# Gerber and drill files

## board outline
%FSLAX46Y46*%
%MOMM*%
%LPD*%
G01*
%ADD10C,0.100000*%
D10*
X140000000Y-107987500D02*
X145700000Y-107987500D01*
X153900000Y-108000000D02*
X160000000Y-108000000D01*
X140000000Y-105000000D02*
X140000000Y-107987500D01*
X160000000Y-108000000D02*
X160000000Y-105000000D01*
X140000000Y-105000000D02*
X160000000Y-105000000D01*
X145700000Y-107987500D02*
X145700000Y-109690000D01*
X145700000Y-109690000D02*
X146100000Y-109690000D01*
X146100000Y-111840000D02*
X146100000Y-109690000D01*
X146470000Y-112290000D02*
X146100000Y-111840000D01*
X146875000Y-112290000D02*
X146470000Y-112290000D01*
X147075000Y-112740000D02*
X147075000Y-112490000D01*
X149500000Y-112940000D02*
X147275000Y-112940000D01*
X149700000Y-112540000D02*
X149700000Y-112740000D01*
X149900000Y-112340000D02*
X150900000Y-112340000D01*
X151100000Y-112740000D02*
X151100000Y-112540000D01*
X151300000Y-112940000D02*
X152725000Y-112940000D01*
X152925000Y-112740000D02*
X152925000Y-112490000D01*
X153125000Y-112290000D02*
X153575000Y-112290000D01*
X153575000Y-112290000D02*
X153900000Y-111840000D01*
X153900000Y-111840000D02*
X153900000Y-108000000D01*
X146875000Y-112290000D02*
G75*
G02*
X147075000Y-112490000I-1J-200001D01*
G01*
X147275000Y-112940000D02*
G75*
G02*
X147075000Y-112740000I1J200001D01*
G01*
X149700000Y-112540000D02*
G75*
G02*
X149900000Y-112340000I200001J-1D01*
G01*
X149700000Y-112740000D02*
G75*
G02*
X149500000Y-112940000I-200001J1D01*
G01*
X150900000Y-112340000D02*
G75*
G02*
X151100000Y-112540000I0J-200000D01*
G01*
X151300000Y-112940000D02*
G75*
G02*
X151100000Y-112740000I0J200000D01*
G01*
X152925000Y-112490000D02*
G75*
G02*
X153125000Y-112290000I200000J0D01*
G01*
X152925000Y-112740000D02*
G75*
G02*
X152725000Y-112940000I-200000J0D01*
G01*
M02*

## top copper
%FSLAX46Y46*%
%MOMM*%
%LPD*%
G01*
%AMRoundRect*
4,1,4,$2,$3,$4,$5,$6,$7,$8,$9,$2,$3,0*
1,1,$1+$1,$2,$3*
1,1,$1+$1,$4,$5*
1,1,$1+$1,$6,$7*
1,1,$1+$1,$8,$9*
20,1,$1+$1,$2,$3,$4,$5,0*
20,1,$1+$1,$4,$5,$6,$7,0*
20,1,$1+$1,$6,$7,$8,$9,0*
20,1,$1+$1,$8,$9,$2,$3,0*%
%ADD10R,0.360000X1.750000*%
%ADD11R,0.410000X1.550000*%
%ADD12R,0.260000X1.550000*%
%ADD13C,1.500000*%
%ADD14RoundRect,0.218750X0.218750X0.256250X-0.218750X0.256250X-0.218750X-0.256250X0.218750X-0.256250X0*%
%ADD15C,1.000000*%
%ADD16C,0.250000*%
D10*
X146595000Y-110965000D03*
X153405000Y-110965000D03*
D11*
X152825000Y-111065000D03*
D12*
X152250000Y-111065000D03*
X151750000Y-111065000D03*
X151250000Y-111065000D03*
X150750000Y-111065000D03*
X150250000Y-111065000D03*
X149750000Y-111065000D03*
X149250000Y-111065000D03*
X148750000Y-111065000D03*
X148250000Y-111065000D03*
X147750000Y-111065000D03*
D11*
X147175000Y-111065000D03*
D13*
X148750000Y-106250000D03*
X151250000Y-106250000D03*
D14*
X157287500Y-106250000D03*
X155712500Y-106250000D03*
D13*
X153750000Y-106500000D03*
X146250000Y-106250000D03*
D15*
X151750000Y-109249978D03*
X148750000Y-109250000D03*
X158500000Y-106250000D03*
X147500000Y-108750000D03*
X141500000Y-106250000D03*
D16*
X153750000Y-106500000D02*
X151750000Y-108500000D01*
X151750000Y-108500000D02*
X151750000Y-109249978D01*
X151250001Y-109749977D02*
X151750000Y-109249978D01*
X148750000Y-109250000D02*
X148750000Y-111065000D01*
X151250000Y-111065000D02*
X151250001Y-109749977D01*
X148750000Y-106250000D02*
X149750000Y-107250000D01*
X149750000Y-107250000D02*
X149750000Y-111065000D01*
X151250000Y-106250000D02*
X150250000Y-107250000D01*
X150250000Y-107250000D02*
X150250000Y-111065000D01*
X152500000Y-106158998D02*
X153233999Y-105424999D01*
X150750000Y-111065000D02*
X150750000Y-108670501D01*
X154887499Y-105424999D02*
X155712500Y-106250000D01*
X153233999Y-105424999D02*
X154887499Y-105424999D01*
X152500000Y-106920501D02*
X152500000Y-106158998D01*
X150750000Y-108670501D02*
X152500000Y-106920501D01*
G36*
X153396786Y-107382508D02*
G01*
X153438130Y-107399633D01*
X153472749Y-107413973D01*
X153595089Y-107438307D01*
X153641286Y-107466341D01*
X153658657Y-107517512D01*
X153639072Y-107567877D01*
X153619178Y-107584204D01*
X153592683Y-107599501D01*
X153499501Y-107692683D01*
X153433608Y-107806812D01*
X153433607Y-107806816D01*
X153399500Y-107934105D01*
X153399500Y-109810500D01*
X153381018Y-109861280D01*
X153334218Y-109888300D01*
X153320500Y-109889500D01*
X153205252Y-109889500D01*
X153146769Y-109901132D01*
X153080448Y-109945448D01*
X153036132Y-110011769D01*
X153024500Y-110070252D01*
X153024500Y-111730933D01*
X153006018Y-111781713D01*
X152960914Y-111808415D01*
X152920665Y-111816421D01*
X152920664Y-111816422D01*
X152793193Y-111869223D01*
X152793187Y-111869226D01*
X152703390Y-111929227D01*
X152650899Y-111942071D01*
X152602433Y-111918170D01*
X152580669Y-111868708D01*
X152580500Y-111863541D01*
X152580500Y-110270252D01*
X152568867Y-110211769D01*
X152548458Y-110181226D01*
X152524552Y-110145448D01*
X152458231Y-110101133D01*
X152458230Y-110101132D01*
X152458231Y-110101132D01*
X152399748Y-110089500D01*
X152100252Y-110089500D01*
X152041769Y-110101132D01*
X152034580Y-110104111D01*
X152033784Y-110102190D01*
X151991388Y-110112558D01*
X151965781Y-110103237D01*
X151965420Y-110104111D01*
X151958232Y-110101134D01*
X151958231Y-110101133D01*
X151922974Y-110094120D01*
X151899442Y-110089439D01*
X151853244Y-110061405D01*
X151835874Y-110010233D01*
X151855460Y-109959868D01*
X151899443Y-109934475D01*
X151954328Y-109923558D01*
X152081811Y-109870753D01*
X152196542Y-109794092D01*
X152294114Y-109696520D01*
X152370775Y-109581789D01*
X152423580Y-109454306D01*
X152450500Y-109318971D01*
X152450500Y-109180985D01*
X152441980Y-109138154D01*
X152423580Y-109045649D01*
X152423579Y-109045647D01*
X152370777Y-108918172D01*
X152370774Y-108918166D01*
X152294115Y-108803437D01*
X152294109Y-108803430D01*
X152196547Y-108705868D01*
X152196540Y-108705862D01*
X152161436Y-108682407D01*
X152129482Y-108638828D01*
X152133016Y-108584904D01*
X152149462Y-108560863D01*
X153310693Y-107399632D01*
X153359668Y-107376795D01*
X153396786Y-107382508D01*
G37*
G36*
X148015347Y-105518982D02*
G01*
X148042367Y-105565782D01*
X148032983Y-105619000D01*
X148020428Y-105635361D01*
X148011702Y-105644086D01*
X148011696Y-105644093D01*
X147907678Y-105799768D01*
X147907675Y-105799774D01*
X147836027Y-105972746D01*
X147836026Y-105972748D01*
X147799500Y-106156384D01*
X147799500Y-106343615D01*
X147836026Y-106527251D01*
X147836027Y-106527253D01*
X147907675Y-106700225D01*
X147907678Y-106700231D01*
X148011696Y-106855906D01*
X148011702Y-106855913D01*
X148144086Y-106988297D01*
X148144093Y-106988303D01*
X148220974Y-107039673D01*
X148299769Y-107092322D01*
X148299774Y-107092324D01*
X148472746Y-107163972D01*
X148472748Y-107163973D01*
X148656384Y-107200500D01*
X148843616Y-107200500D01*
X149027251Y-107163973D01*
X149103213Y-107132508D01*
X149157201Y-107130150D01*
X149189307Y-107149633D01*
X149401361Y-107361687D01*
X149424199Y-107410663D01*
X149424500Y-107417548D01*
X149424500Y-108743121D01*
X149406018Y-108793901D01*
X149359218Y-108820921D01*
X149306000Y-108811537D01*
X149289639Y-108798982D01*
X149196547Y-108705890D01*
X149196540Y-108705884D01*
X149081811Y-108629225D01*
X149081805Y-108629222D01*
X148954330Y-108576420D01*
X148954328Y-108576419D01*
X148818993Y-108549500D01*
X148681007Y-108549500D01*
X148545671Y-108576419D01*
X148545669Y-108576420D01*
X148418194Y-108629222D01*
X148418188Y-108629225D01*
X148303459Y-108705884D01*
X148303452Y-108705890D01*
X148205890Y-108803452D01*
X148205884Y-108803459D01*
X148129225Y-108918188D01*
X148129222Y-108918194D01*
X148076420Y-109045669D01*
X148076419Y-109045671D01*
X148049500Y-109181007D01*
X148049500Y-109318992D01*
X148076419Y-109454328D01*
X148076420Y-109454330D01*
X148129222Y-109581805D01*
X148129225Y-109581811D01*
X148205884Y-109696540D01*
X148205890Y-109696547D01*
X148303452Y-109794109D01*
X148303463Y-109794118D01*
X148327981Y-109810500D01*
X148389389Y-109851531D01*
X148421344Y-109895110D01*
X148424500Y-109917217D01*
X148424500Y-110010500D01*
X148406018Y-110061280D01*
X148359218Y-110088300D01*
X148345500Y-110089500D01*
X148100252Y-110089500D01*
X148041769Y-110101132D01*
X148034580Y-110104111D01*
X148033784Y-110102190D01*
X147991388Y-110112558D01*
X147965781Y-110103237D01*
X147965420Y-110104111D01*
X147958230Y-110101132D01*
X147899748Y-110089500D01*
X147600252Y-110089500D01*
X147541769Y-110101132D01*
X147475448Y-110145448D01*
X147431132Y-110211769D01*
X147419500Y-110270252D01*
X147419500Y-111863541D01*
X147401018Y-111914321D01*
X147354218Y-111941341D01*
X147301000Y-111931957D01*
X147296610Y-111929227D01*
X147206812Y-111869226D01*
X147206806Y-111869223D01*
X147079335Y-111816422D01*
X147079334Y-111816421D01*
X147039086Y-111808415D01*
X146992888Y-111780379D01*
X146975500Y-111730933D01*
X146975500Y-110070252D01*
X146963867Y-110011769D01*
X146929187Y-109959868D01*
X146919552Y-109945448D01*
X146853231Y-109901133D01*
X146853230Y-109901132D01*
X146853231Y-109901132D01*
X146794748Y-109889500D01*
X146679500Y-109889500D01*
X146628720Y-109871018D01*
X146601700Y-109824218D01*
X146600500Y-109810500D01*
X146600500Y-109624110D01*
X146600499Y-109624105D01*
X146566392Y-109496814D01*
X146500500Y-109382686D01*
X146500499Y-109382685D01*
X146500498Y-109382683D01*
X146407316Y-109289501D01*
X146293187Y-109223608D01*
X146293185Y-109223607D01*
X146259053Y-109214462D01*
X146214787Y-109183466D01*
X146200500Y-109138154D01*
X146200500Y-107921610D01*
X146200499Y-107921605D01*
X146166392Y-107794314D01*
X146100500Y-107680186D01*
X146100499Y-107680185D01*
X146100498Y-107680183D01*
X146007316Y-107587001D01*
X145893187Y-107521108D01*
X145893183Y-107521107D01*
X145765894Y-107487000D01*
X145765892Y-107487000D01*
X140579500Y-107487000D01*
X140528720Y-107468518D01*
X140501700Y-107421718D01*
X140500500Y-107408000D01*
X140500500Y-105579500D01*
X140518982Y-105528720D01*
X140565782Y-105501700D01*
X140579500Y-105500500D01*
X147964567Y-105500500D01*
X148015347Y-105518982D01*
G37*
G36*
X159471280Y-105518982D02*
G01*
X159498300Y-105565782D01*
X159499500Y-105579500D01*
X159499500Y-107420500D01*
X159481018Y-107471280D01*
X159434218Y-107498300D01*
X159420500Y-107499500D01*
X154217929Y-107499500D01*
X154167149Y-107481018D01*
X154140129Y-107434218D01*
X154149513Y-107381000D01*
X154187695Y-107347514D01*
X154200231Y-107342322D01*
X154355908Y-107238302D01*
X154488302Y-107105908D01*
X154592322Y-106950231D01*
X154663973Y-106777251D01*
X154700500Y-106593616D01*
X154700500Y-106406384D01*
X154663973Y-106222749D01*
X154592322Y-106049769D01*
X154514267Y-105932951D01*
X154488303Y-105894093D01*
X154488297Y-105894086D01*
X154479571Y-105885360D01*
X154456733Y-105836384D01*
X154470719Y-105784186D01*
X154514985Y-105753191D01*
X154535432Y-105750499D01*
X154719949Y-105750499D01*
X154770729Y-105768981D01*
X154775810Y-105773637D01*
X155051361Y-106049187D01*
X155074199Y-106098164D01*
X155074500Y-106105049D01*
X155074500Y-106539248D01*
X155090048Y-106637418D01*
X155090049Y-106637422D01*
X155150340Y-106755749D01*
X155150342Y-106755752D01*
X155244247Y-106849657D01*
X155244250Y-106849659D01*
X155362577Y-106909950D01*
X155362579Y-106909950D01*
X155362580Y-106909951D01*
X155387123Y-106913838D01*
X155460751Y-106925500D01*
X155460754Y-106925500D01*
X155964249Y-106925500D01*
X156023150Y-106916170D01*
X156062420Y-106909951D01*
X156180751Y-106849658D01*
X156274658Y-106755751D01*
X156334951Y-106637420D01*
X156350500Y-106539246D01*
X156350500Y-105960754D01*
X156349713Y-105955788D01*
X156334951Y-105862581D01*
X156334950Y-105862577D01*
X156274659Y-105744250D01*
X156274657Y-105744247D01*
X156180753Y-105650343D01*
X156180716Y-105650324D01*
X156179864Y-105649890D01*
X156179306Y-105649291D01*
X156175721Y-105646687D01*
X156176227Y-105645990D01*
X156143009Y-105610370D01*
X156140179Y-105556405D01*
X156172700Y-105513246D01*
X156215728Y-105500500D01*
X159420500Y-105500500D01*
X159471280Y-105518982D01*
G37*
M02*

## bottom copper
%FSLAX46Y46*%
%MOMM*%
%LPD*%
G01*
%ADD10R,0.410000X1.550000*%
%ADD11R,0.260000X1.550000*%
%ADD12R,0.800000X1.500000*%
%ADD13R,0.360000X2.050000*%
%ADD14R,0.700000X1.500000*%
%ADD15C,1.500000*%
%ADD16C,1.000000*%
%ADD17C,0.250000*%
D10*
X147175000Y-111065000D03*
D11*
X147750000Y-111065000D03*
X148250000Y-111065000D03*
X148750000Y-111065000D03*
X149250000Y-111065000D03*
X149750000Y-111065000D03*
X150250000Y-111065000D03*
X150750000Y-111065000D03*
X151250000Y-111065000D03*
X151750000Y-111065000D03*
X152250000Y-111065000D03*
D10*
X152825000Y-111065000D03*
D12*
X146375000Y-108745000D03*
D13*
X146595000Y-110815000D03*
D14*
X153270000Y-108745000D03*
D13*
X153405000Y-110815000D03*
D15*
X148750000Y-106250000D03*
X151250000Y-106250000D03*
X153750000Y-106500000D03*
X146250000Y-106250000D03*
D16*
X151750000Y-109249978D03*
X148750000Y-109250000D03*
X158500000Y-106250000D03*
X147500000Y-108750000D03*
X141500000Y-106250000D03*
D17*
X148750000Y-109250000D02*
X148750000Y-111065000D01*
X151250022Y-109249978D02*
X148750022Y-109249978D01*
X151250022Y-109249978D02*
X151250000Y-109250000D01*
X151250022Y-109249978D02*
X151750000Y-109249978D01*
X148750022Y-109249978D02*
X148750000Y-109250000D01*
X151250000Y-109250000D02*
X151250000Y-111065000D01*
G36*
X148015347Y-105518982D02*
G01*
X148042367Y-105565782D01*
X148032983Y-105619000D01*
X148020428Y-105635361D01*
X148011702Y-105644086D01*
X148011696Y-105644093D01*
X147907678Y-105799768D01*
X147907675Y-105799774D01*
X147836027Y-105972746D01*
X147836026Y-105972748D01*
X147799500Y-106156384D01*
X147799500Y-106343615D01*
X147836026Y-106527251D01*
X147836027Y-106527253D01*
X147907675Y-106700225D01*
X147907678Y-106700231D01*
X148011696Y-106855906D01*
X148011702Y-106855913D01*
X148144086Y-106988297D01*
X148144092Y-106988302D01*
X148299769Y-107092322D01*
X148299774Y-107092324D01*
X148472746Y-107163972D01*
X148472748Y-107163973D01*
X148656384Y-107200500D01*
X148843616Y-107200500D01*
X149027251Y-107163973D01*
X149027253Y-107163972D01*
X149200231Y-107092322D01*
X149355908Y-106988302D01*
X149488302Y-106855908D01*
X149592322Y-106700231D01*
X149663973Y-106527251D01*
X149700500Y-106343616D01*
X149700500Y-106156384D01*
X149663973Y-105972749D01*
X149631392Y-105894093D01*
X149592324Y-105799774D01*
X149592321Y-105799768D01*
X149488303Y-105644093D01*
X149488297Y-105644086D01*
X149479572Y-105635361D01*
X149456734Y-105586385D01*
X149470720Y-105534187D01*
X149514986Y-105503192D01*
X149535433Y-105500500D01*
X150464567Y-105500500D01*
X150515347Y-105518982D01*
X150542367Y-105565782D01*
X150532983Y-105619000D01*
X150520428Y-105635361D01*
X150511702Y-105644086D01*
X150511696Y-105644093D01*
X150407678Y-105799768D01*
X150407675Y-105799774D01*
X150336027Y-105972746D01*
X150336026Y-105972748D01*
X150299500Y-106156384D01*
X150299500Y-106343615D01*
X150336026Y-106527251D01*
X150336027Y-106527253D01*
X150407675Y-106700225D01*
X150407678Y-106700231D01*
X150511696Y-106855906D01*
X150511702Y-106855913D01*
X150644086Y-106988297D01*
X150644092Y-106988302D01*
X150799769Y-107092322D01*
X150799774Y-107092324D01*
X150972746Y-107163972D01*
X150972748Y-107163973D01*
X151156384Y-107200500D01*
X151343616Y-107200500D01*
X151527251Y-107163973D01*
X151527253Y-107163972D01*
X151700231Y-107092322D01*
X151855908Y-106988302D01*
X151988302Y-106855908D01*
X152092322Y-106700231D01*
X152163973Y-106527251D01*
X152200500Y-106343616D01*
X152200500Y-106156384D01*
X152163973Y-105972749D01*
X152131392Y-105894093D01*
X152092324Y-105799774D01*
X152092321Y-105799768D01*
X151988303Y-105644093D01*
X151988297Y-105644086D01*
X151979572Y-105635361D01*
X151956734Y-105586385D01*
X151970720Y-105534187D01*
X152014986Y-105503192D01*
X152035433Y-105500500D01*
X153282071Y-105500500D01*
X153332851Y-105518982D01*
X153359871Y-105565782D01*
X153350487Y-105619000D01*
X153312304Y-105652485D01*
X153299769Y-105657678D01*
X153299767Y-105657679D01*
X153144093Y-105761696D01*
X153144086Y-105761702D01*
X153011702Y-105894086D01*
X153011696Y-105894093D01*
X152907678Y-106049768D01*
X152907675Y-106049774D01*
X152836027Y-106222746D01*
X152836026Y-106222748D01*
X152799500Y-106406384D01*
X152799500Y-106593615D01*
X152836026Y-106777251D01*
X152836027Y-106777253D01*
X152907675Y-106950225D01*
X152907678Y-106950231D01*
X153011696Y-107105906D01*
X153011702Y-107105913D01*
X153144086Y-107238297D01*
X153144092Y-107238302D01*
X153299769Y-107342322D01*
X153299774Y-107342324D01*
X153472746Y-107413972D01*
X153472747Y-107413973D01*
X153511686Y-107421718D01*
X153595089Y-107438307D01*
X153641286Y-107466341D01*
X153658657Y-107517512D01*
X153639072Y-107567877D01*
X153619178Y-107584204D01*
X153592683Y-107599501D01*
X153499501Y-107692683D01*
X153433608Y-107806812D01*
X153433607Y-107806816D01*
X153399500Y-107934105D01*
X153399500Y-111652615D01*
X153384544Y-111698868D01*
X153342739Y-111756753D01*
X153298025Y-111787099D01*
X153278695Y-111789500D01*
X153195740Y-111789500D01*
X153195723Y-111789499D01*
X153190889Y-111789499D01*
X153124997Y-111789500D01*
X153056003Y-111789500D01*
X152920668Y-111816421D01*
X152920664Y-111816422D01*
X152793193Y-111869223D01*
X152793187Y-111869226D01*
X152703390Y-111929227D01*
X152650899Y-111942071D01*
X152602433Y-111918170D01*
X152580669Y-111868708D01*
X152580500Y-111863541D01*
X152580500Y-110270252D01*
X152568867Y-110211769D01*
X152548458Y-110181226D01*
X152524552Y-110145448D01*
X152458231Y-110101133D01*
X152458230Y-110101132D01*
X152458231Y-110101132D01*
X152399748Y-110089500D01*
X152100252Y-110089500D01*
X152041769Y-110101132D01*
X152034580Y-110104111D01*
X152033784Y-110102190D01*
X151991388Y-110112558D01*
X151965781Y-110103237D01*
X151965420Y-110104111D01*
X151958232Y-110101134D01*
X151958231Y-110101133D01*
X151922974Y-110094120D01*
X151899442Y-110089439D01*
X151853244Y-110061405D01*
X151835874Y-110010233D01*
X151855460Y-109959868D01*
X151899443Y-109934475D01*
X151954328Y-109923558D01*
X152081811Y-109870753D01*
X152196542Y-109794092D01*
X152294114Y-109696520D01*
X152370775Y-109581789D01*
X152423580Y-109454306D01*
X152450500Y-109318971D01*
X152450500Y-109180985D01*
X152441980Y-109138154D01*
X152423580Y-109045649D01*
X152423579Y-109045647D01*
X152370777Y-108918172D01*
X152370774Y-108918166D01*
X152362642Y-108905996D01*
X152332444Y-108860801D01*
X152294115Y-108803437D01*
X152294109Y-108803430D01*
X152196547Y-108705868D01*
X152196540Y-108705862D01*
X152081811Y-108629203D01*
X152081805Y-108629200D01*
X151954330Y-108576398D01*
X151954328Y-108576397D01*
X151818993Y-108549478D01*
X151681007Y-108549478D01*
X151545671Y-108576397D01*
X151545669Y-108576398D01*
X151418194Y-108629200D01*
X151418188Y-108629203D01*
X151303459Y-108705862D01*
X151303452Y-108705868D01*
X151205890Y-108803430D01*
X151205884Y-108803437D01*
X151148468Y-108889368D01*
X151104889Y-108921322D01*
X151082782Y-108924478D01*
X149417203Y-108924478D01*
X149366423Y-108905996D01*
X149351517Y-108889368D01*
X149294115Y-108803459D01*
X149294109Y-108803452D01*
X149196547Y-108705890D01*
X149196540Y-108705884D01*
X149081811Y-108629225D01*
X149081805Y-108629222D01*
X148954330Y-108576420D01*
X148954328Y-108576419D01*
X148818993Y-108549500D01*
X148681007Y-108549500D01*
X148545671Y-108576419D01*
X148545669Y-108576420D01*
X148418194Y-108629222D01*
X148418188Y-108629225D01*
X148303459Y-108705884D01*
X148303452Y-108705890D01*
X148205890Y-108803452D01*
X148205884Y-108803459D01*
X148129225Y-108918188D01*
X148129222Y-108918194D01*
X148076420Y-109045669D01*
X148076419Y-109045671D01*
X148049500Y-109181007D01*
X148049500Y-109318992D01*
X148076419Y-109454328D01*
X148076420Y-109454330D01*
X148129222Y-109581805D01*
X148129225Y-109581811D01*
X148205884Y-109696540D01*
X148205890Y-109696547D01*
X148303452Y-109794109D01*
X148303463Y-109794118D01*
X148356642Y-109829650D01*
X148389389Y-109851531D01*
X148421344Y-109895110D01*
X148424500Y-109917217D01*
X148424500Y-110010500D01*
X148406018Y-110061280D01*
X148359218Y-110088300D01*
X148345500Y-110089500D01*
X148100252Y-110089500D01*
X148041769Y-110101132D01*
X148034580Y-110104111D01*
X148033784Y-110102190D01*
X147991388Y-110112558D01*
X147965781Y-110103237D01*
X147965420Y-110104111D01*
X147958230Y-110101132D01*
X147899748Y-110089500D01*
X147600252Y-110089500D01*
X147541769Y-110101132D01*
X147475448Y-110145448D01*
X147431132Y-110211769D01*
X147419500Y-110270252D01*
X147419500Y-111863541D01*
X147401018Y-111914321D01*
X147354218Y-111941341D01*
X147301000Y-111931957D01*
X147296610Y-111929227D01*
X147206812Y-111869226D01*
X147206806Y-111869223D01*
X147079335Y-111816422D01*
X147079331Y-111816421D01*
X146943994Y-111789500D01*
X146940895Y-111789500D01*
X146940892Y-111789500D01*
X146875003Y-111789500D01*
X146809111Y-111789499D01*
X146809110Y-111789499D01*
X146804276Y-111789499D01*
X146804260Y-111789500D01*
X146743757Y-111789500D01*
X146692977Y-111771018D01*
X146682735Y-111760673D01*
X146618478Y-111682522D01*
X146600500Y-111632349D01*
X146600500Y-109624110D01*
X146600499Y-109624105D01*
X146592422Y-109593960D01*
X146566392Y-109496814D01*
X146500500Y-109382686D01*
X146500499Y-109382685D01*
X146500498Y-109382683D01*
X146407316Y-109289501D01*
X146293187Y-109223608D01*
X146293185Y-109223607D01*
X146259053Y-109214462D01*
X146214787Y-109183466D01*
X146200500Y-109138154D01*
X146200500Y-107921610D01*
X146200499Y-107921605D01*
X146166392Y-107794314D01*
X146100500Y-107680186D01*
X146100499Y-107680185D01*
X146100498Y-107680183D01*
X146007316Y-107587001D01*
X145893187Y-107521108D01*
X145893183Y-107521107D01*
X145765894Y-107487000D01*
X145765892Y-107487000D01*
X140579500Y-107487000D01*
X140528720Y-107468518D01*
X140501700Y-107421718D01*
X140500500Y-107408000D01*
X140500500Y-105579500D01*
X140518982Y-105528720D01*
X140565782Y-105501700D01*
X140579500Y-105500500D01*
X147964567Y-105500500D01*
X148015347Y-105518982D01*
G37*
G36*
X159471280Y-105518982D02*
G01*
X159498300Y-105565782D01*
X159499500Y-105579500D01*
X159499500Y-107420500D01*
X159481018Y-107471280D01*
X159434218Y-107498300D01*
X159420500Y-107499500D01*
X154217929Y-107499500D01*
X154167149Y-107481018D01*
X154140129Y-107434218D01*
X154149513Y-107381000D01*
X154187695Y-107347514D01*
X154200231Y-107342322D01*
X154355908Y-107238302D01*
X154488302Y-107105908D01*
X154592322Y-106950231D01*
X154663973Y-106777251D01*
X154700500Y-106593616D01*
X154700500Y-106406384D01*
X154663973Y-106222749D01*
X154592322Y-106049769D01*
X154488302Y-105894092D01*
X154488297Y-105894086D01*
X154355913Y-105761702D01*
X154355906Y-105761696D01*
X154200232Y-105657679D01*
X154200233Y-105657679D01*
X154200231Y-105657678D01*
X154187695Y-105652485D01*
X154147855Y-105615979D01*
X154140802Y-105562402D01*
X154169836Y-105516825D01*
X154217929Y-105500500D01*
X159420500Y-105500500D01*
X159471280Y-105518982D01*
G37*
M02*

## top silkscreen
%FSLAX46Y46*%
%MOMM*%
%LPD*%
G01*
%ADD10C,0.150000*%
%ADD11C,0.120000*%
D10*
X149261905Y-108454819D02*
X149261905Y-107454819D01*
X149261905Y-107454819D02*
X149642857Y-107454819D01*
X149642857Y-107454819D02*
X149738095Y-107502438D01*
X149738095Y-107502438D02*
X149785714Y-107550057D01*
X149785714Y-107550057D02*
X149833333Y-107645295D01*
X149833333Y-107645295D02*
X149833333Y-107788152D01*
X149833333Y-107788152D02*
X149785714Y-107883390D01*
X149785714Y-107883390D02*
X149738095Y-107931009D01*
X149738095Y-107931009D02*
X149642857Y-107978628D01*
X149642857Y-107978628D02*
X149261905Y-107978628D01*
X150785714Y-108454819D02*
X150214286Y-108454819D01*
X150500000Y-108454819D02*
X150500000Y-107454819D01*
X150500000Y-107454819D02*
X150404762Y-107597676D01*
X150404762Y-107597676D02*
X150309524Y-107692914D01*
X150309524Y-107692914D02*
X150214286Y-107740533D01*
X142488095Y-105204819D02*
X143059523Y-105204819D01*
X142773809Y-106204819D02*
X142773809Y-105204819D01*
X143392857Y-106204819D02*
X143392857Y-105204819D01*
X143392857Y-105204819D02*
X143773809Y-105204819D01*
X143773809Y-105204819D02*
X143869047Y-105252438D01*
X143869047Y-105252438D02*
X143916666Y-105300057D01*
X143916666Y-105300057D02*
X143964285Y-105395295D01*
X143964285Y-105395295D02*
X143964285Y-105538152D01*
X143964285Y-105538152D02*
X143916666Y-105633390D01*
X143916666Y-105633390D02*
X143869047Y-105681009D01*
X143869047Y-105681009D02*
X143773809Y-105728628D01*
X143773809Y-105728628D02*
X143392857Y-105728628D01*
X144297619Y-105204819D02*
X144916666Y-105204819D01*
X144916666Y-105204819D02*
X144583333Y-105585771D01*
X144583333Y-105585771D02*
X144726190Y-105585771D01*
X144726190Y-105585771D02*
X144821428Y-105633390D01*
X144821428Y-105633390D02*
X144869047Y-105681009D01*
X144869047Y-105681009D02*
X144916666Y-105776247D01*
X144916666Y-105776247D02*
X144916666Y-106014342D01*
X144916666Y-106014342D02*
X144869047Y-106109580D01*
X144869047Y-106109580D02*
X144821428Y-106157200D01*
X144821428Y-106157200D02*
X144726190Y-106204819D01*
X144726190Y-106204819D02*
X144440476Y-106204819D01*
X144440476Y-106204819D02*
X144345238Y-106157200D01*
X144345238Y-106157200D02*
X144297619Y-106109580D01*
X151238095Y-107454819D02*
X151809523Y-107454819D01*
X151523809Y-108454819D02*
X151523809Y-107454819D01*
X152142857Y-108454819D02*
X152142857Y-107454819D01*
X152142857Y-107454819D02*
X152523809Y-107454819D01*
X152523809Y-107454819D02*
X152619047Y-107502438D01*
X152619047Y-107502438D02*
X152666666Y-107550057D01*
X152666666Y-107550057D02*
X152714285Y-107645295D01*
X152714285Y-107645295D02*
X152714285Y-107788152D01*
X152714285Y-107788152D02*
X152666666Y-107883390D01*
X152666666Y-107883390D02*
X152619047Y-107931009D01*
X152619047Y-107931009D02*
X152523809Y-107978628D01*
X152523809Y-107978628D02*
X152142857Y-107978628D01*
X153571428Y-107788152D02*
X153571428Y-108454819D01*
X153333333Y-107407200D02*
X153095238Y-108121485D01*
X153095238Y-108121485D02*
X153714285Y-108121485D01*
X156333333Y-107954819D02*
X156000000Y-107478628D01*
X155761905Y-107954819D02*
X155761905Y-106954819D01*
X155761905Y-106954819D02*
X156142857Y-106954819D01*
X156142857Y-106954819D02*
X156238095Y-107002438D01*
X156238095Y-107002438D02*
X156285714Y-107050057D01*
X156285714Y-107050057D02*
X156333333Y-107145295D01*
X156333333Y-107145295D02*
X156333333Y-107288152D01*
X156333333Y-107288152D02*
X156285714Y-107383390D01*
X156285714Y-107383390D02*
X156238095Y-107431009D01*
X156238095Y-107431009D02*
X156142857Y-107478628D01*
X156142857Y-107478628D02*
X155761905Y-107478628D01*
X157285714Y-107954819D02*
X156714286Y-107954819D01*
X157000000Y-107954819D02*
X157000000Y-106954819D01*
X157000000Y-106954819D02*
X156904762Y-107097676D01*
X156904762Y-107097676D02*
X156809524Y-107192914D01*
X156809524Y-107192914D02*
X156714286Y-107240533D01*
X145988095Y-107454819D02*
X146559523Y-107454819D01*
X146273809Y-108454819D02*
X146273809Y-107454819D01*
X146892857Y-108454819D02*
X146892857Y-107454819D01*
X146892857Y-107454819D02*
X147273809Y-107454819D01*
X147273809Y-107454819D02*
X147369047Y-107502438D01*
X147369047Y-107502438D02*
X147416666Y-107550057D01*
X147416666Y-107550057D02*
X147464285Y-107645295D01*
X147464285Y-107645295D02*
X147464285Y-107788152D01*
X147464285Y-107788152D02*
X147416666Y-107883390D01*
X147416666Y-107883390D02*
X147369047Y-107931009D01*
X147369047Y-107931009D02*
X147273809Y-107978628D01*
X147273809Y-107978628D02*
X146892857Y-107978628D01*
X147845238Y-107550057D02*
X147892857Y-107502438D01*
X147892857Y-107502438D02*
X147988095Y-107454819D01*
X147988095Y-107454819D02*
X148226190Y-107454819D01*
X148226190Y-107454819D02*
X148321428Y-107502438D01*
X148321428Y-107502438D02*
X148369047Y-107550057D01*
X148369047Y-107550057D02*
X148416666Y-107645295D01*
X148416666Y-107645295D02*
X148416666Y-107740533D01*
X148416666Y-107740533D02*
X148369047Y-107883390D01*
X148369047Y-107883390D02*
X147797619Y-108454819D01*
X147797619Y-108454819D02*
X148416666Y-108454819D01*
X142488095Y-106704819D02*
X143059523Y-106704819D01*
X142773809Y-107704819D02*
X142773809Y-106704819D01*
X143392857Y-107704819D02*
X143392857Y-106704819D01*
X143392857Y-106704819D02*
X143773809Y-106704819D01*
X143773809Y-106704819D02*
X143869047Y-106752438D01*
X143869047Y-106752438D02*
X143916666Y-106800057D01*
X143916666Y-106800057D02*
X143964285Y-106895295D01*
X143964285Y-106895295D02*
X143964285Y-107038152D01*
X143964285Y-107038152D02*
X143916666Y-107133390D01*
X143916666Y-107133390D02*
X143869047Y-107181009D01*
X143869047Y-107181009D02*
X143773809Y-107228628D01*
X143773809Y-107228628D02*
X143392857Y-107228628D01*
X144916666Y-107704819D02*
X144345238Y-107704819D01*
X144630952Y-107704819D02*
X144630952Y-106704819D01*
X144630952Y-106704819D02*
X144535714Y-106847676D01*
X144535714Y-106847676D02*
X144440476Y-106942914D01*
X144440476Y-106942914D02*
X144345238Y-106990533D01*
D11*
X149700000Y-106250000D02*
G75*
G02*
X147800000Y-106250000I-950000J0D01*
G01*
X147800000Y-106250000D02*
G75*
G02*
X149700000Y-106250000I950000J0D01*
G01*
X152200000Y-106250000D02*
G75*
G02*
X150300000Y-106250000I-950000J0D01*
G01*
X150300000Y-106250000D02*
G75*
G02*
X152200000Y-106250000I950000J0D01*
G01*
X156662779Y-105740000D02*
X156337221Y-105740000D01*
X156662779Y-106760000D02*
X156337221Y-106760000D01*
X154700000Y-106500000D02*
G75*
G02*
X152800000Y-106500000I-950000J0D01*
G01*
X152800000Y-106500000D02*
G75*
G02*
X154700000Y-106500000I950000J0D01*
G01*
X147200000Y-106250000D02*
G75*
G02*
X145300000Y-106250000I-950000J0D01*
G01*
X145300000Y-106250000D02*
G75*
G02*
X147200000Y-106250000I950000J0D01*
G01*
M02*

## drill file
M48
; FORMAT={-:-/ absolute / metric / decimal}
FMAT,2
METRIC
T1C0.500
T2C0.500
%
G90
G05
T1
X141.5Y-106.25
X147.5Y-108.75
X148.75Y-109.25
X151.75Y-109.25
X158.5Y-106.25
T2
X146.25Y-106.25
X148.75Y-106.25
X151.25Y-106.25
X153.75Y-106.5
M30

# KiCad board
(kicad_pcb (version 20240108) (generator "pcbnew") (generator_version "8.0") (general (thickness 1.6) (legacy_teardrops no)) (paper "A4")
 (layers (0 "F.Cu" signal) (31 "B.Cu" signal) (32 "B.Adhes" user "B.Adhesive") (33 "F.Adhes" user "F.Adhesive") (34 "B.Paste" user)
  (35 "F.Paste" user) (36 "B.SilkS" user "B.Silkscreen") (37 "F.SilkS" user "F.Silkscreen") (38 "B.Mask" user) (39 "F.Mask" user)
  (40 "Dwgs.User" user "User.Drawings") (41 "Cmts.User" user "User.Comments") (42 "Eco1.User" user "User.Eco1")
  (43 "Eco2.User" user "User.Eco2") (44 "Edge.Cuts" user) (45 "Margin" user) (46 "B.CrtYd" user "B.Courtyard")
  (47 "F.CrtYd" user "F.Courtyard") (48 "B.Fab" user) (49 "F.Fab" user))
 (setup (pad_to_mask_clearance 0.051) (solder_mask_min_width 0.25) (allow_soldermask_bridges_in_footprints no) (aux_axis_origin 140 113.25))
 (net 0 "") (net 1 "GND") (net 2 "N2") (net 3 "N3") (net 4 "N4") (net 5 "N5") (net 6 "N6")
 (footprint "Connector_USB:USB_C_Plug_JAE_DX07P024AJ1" (layer "F.Cu") (at 150 109.9175)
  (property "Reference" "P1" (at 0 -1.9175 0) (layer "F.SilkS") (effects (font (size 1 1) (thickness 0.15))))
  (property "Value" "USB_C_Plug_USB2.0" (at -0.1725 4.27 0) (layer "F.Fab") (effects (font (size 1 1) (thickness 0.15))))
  (fp_line (start -4.3 -1.93) (end -4.3 -0.2275) (stroke (width 0.1) (type solid)) (layer "Edge.Cuts"))
  (fp_line (start -4.3 -0.2275) (end -3.9 -0.2275) (stroke (width 0.1) (type solid)) (layer "Edge.Cuts"))
  (fp_line (start -3.9 1.9225) (end -3.9 -0.2275) (stroke (width 0.1) (type solid)) (layer "Edge.Cuts"))
  (fp_line (start -3.53 2.3725) (end -3.9 1.9225) (stroke (width 0.1) (type solid)) (layer "Edge.Cuts"))
  (fp_line (start -3.125 2.3725) (end -3.53 2.3725) (stroke (width 0.1) (type solid)) (layer "Edge.Cuts"))
  (fp_line (start -2.925 2.8225) (end -2.925 2.5725) (stroke (width 0.1) (type solid)) (layer "Edge.Cuts"))
  (fp_line (start -0.5 3.0225) (end -2.725 3.0225) (stroke (width 0.1) (type solid)) (layer "Edge.Cuts"))
  (fp_line (start -0.3 2.6225) (end -0.3 2.8225) (stroke (width 0.1) (type solid)) (layer "Edge.Cuts"))
  (fp_line (start -0.1 2.4225) (end 0.9 2.4225) (stroke (width 0.1) (type solid)) (layer "Edge.Cuts"))
  (fp_line (start 1.1 2.8225) (end 1.1 2.6225) (stroke (width 0.1) (type solid)) (layer "Edge.Cuts"))
  (fp_line (start 1.3 3.0225) (end 2.725 3.0225) (stroke (width 0.1) (type solid)) (layer "Edge.Cuts"))
  (fp_line (start 2.925 2.8225) (end 2.925 2.5725) (stroke (width 0.1) (type solid)) (layer "Edge.Cuts"))
  (fp_line (start 3.125 2.3725) (end 3.575 2.3725) (stroke (width 0.1) (type solid)) (layer "Edge.Cuts"))
  (fp_line (start 3.575 2.3725) (end 3.9 1.9225) (stroke (width 0.1) (type solid)) (layer "Edge.Cuts"))
  (fp_line (start 3.9 1.9225) (end 3.9 -1.9175) (stroke (width 0.1) (type solid)) (layer "Edge.Cuts"))
  (fp_arc (start -3.125 2.3725) (mid -2.983579 2.431079) (end -2.925 2.5725) (stroke (width 0.1) (type solid)) (layer "Edge.Cuts"))
  (fp_arc (start -2.725 3.0225) (mid -2.866421 2.963921) (end -2.925 2.8225) (stroke (width 0.1) (type solid)) (layer "Edge.Cuts"))
  (fp_arc (start -0.3 2.6225) (mid -0.241421 2.481079) (end -0.1 2.4225) (stroke (width 0.1) (type solid)) (layer "Edge.Cuts"))
  (fp_arc (start -0.3 2.8225) (mid -0.358579 2.963921) (end -0.5 3.0225) (stroke (width 0.1) (type solid)) (layer "Edge.Cuts"))
  (fp_arc (start 0.9 2.4225) (mid 1.041421 2.481079) (end 1.1 2.6225) (stroke (width 0.1) (type solid)) (layer "Edge.Cuts"))
  (fp_arc (start 1.3 3.0225) (mid 1.158579 2.963921) (end 1.1 2.8225) (stroke (width 0.1) (type solid)) (layer "Edge.Cuts"))
  (fp_arc (start 2.925 2.5725) (mid 2.983579 2.431079) (end 3.125 2.3725) (stroke (width 0.1) (type solid)) (layer "Edge.Cuts"))
  (fp_arc (start 2.925 2.8225) (mid 2.866421 2.963921) (end 2.725 3.0225) (stroke (width 0.1) (type solid)) (layer "Edge.Cuts"))
  (pad "" smd rect (at -3.405 1.0475) (size 0.36 1.75) (layers "F.Cu" "F.Mask"))
  (pad "" smd rect (at 3.405 1.0475) (size 0.36 1.75) (layers "F.Cu" "F.Mask"))
  (pad "A1" smd rect (at 2.825 1.1475) (size 0.41 1.55) (layers "F.Cu" "F.Paste" "F.Mask") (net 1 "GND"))
  (pad "A2" smd rect (at 2.25 1.1475) (size 0.26 1.55) (layers "F.Cu" "F.Paste" "F.Mask"))
  (pad "A3" smd rect (at 1.75 1.1475) (size 0.26 1.55) (layers "F.Cu" "F.Paste" "F.Mask"))
  (pad "A4" smd rect (at 1.25 1.1475) (size 0.26 1.55) (layers "F.Cu" "F.Paste" "F.Mask") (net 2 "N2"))
  (pad "A5" smd rect (at 0.75 1.1475) (size 0.26 1.55) (layers "F.Cu" "F.Paste" "F.Mask") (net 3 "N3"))
  (pad "A6" smd rect (at 0.25 1.1475 180) (size 0.26 1.55) (layers "F.Cu" "F.Paste" "F.Mask") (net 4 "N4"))
  (pad "A7" smd rect (at -0.25 1.1475 180) (size 0.26 1.55) (layers "F.Cu" "F.Paste" "F.Mask") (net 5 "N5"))
  (pad "A8" smd rect (at -0.75 1.1475) (size 0.26 1.55) (layers "F.Cu" "F.Paste" "F.Mask"))
  (pad "A9" smd rect (at -1.25 1.1475) (size 0.26 1.55) (layers "F.Cu" "F.Paste" "F.Mask") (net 2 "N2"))
  (pad "A10" smd rect (at -1.75 1.1475) (size 0.26 1.55) (layers "F.Cu" "F.Paste" "F.Mask"))
  (pad "A11" smd rect (at -2.25 1.1475) (size 0.26 1.55) (layers "F.Cu" "F.Paste" "F.Mask"))
  (pad "A12" smd rect (at -2.825 1.1475) (size 0.41 1.55) (layers "F.Cu" "F.Paste" "F.Mask") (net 1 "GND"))
  (pad "B1" smd rect (at -2.825 1.1475) (size 0.41 1.55) (layers "B.Cu" "B.Paste" "B.Mask") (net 1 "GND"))
  (pad "B2" smd rect (at -2.25 1.1475) (size 0.26 1.55) (layers "B.Cu" "B.Paste" "B.Mask"))
  (pad "B3" smd rect (at -1.75 1.1475) (size 0.26 1.55) (layers "B.Cu" "B.Paste" "B.Mask"))
  (pad "B4" smd rect (at -1.25 1.1475) (size 0.26 1.55) (layers "B.Cu" "B.Paste" "B.Mask") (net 2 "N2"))
  (pad "B5" smd rect (at -0.75 1.1475) (size 0.26 1.55) (layers "B.Cu" "B.Paste" "B.Mask") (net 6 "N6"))
  (pad "B6" smd rect (at -0.25 1.1475 180) (size 0.26 1.55) (layers "B.Cu" "B.Paste" "B.Mask"))
  (pad "B7" smd rect (at 0.25 1.1475) (size 0.26 1.55) (layers "B.Cu" "B.Paste" "B.Mask"))
  (pad "B8" smd rect (at 0.75 1.1475) (size 0.26 1.55) (layers "B.Cu" "B.Paste" "B.Mask"))
  (pad "B9" smd rect (at 1.25 1.1475) (size 0.26 1.55) (layers "B.Cu" "B.Paste" "B.Mask") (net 2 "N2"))
  (pad "B10" smd rect (at 1.75 1.1475) (size 0.26 1.55) (layers "B.Cu" "B.Paste" "B.Mask"))
  (pad "B11" smd rect (at 2.25 1.1475) (size 0.26 1.55) (layers "B.Cu" "B.Paste" "B.Mask"))
  (pad "B12" smd rect (at 2.825 1.1475) (size 0.41 1.55) (layers "B.Cu" "B.Paste" "B.Mask") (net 1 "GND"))
  (pad "S1" smd rect (at -3.625 -1.1725) (size 0.8 1.5) (layers "B.Cu" "B.Paste" "B.Mask") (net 1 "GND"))
  (pad "S1" smd rect (at -3.405 0.8975) (size 0.36 2.05) (layers "B.Cu" "B.Paste" "B.Mask") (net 1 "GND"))
  (pad "S1" smd rect (at 3.27 -1.1725 180) (size 0.7 1.5) (layers "B.Cu" "B.Paste" "B.Mask") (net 1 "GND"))
  (pad "S1" smd rect (at 3.405 0.8975) (size 0.36 2.05) (layers "B.Cu" "B.Paste" "B.Mask") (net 1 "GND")))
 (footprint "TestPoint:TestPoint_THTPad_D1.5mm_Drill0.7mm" (layer "F.Cu") (at 148.75 106.25)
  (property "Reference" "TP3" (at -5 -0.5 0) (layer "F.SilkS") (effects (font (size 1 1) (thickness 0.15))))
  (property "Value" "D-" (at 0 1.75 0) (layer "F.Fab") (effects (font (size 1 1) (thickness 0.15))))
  (fp_circle (center 0 0) (end 0 0.95) (stroke (width 0.12) (type solid)) (fill none) (layer "F.SilkS"))
  (pad "1" thru_hole circle (at 0 0) (size 1.5 1.5) (drill 0.5) (layers "*.Cu" "*.Mask") (remove_unused_layers no) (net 5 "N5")))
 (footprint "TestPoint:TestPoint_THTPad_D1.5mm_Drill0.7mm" (layer "F.Cu") (at 151.25 106.25)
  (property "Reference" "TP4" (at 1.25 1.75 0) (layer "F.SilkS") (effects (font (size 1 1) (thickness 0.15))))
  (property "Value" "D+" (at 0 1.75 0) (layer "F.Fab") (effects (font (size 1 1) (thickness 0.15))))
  (fp_circle (center 0 0) (end 0 0.95) (stroke (width 0.12) (type solid)) (fill none) (layer "F.SilkS"))
  (pad "1" thru_hole circle (at 0 0) (size 1.5 1.5) (drill 0.5) (layers "*.Cu" "*.Mask") (remove_unused_layers no) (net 4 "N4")))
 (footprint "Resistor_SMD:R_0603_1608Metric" (layer "F.Cu") (at 156.5 106.25 180)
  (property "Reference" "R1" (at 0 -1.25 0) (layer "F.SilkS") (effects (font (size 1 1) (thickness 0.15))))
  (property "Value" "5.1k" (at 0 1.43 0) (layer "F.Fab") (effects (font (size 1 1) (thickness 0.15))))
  (fp_line (start -0.162779 0.51) (end 0.162779 0.51) (stroke (width 0.12) (type solid)) (layer "F.SilkS"))
  (fp_line (start -0.162779 -0.51) (end 0.162779 -0.51) (stroke (width 0.12) (type solid)) (layer "F.SilkS"))
  (pad "1" smd roundrect (at -0.7875 0 180) (size 0.875 0.95) (layers "F.Cu" "F.Paste" "F.Mask") (roundrect_rratio 0.25) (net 1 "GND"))
  (pad "2" smd roundrect (at 0.7875 0 180) (size 0.875 0.95) (layers "F.Cu" "F.Paste" "F.Mask") (roundrect_rratio 0.25) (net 3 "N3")))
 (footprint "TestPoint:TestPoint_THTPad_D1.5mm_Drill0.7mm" (layer "F.Cu") (at 153.75 106.5)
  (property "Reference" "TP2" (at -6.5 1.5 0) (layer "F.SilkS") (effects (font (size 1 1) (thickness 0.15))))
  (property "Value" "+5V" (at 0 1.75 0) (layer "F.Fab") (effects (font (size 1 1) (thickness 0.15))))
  (fp_circle (center 0 0) (end 0 0.95) (stroke (width 0.12) (type solid)) (fill none) (layer "F.SilkS"))
  (pad "1" thru_hole circle (at 0 0) (size 1.5 1.5) (drill 0.5) (layers "*.Cu" "*.Mask") (remove_unused_layers no) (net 2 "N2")))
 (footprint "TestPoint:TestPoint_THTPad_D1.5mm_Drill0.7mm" (layer "F.Cu") (at 146.25 106.25)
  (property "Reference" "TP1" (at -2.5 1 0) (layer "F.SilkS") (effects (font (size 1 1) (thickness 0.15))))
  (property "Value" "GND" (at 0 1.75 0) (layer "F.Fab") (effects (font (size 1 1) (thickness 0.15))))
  (fp_circle (center 0 0) (end 0 0.95) (stroke (width 0.12) (type solid)) (fill none) (layer "F.SilkS"))
  (pad "1" thru_hole circle (at 0 0) (size 1.5 1.5) (drill 0.5) (layers "*.Cu" "*.Mask") (remove_unused_layers no) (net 1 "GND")))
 (gr_line (start 140 107.9875) (end 145.7 107.9875) (stroke (width 0.1) (type solid)) (layer "Edge.Cuts"))
 (gr_line (start 153.9 108) (end 160 108) (stroke (width 0.1) (type solid)) (layer "Edge.Cuts"))
 (gr_line (start 140 105) (end 140 107.9875) (stroke (width 0.1) (type solid)) (layer "Edge.Cuts"))
 (gr_line (start 160 108) (end 160 105) (stroke (width 0.1) (type solid)) (layer "Edge.Cuts"))
 (gr_line (start 140 105) (end 160 105) (stroke (width 0.1) (type solid)) (layer "Edge.Cuts"))
 (segment (start 153.75 106.5) (end 151.75 108.5) (width 0.25) (layer "F.Cu") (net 2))
 (segment (start 151.75 108.5) (end 151.75 109.249978) (width 0.25) (layer "F.Cu") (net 2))
 (segment (start 151.250001 109.749977) (end 151.75 109.249978) (width 0.25) (layer "F.Cu") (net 2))
 (segment (start 148.75 109.25) (end 148.75 111.065) (width 0.25) (layer "F.Cu") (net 2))
 (segment (start 151.25 111.065) (end 151.250001 109.749977) (width 0.25) (layer "F.Cu") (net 2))
 (via (at 151.75 109.249978) (size 1) (drill 0.5) (layers "F.Cu" "B.Cu") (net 2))
 (via (at 148.75 109.25) (size 1) (drill 0.5) (layers "F.Cu" "B.Cu") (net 2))
 (segment (start 148.75 109.25) (end 148.75 111.065) (width 0.25) (layer "B.Cu") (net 2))
 (segment (start 151.250022 109.249978) (end 148.750022 109.249978) (width 0.25) (layer "B.Cu") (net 2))
 (segment (start 151.250022 109.249978) (end 151.25 109.25) (width 0.25) (layer "B.Cu") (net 2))
 (segment (start 151.250022 109.249978) (end 151.75 109.249978) (width 0.25) (layer "B.Cu") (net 2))
 (segment (start 148.750022 109.249978) (end 148.75 109.25) (width 0.25) (layer "B.Cu") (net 2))
 (segment (start 151.25 109.25) (end 151.25 111.065) (width 0.25) (layer "B.Cu") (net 2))
 (segment (start 148.75 106.25) (end 149.75 107.25) (width 0.25) (layer "F.Cu") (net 5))
 (segment (start 149.75 107.25) (end 149.75 111.065) (width 0.25) (layer "F.Cu") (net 5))
 (segment (start 151.25 106.25) (end 150.25 107.25) (width 0.25) (layer "F.Cu") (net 4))
 (segment (start 150.25 107.25) (end 150.25 111.065) (width 0.25) (layer "F.Cu") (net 4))
 (segment (start 152.5 106.158998) (end 153.233999 105.424999) (width 0.25) (layer "F.Cu") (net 3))
 (segment (start 150.75 111.065) (end 150.75 108.670501) (width 0.25) (layer "F.Cu") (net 3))
 (segment (start 154.887499 105.424999) (end 155.7125 106.25) (width 0.25) (layer "F.Cu") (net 3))
 (segment (start 153.233999 105.424999) (end 154.887499 105.424999) (width 0.25) (layer "F.Cu") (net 3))
 (segment (start 152.5 106.920501) (end 152.5 106.158998) (width 0.25) (layer "F.Cu") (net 3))
 (segment (start 150.75 108.670501) (end 152.5 106.920501) (width 0.25) (layer "F.Cu") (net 3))
 (via (at 158.5 106.25) (size 1) (drill 0.5) (layers "F.Cu" "B.Cu") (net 1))
 (via (at 147.5 108.75) (size 1) (drill 0.5) (layers "F.Cu" "B.Cu") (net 1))
 (via (at 141.5 106.25) (size 1) (drill 0.5) (layers "F.Cu" "B.Cu") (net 1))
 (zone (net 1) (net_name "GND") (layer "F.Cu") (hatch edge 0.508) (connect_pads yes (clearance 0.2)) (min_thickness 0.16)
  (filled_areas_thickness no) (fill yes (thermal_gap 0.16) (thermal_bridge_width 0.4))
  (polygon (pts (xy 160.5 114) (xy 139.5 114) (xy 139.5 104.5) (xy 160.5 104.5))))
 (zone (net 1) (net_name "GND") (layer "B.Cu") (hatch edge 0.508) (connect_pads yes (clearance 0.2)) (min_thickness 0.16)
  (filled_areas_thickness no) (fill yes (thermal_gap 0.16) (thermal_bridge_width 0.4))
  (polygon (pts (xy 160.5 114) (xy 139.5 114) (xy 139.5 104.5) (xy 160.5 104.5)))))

